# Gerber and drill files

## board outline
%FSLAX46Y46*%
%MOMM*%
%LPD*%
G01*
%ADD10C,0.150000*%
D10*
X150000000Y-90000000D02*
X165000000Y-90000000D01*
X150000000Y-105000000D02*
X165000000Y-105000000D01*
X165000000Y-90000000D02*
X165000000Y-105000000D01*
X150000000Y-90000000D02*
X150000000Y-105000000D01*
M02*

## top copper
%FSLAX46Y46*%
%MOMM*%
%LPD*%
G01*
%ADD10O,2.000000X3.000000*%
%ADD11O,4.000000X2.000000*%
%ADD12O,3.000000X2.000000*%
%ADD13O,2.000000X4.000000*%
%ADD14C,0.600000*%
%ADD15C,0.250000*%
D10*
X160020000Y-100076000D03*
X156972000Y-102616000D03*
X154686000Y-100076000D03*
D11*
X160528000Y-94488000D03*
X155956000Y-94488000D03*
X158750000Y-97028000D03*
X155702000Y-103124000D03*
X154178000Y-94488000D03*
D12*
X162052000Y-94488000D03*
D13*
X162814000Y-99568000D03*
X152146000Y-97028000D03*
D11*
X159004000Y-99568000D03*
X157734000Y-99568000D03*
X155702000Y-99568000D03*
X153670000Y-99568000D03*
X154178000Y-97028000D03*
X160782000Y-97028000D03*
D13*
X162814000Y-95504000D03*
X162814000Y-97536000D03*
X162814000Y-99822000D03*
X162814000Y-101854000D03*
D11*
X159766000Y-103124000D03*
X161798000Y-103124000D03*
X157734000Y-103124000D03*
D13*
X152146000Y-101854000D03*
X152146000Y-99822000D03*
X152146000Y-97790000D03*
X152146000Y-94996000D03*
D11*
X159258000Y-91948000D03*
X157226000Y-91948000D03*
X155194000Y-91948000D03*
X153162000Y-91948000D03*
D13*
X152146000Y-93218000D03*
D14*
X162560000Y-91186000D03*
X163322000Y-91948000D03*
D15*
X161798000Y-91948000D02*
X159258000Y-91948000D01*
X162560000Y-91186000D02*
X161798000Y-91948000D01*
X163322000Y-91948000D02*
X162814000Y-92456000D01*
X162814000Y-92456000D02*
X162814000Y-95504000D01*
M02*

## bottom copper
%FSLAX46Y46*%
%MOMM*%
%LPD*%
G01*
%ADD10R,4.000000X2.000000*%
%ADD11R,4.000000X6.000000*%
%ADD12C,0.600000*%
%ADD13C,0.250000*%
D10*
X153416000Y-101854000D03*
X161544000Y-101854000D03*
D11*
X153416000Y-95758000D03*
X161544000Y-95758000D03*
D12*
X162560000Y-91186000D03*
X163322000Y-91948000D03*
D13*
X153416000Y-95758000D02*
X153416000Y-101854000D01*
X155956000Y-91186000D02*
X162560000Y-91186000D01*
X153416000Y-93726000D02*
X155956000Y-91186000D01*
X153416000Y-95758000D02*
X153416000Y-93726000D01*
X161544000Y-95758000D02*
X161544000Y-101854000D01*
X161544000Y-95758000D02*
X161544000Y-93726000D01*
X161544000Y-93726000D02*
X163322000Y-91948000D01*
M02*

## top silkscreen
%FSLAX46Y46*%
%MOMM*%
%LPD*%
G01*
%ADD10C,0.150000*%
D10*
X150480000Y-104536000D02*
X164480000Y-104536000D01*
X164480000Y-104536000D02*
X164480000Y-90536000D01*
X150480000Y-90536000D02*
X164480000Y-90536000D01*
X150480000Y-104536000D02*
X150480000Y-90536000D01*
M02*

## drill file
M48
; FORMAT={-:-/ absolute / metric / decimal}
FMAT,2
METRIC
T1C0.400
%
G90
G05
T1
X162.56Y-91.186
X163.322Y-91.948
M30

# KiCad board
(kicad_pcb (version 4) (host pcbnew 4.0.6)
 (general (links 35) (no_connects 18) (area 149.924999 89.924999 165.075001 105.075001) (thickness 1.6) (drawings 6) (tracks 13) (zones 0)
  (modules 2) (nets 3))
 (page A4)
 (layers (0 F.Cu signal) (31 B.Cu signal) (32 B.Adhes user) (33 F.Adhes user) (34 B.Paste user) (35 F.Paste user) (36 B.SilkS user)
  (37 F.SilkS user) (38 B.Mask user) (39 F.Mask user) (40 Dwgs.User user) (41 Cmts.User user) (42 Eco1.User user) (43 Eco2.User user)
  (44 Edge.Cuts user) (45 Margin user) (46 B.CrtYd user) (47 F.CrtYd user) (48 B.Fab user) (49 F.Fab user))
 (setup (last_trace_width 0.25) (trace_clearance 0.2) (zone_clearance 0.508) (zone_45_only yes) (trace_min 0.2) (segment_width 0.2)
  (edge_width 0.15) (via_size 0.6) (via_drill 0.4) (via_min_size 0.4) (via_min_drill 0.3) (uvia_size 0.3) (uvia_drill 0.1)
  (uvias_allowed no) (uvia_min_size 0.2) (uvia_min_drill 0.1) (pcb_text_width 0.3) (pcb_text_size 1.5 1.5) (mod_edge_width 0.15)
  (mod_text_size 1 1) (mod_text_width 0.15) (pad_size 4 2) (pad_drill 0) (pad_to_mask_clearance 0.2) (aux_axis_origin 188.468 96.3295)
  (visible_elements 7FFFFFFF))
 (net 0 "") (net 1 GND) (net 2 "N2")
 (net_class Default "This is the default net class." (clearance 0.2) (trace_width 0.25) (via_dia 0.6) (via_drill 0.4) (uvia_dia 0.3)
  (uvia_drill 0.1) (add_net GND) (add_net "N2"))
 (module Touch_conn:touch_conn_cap (layer B.Cu) (at 157.48 97.79 90)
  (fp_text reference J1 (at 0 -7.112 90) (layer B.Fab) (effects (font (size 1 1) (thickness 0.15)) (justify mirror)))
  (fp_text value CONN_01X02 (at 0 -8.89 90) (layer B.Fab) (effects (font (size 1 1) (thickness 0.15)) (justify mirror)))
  (pad 2 smd rect (at -4.064 -4.064 90) (size 2 4) (layers B.Cu B.Paste B.Mask) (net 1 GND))
  (pad 1 smd rect (at -4.064 4.064 90) (size 2 4) (layers B.Cu B.Paste B.Mask) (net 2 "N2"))
  (pad 2 smd rect (at 2.032 -4.064 90) (size 6 4) (layers B.Cu B.Paste B.Mask) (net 1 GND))
  (pad 1 smd rect (at 2.032 4.064 90) (size 6 4) (layers B.Cu B.Paste B.Mask) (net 2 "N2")))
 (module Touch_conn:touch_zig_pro (layer F.Cu) (at 157.48 97.536)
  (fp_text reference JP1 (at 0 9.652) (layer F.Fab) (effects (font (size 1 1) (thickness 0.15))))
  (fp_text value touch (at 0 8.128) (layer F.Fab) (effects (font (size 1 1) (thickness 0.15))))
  (fp_line (start -7 7) (end 7 7) (layer F.SilkS) (width 0.15))
  (fp_line (start 7 7) (end 7 -7) (layer F.SilkS) (width 0.15))
  (fp_line (start -7 -7) (end 7 -7) (layer F.SilkS) (width 0.15))
  (fp_line (start -7 7) (end -7 -7) (layer F.SilkS) (width 0.15))
  (pad 1 smd oval (at 2.54 2.54) (size 2 3) (layers F.Cu F.Paste F.Mask) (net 1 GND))
  (pad 2 smd oval (at -0.508 5.08) (size 2 3) (layers F.Cu F.Paste F.Mask) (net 2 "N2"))
  (pad 1 smd oval (at -2.794 2.54) (size 2 3) (layers F.Cu F.Paste F.Mask) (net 1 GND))
  (pad 2 smd oval (at 3.048 -3.048) (size 4 2) (layers F.Cu F.Paste F.Mask) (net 2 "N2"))
  (pad 1 smd oval (at -1.524 -3.048) (size 4 2) (layers F.Cu F.Paste F.Mask) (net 1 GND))
  (pad 2 smd oval (at 1.27 -0.508) (size 4 2) (layers F.Cu F.Paste F.Mask) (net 2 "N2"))
  (pad 2 smd oval (at -1.778 5.588) (size 4 2) (layers F.Cu F.Paste F.Mask) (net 2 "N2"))
  (pad 1 smd oval (at -3.302 -3.048) (size 4 2) (layers F.Cu F.Paste F.Mask) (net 1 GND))
  (pad 2 smd oval (at 4.572 -3.048) (size 3 2) (layers F.Cu F.Paste F.Mask) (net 2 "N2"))
  (pad 2 smd oval (at 5.334 2.032) (size 2 4) (layers F.Cu F.Paste F.Mask) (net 2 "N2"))
  (pad 1 smd oval (at -5.334 -0.508) (size 2 4) (layers F.Cu F.Paste F.Mask) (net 1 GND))
  (pad 1 smd oval (at 1.524 2.032) (size 4 2) (layers F.Cu F.Paste F.Mask) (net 1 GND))
  (pad 1 smd oval (at 0.254 2.032) (size 4 2) (layers F.Cu F.Paste F.Mask) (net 1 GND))
  (pad 1 smd oval (at -1.778 2.032) (size 4 2) (layers F.Cu F.Paste F.Mask) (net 1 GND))
  (pad 1 smd oval (at -3.81 2.032) (size 4 2) (layers F.Cu F.Paste F.Mask) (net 1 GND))
  (pad 1 smd oval (at -3.302 -0.508) (size 4 2) (layers F.Cu F.Paste F.Mask) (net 1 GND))
  (pad 2 smd oval (at 3.302 -0.508) (size 4 2) (layers F.Cu F.Paste F.Mask) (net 2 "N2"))
  (pad 2 smd oval (at 5.334 -2.032) (size 2 4) (layers F.Cu F.Paste F.Mask) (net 2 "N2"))
  (pad 2 smd oval (at 5.334 0) (size 2 4) (layers F.Cu F.Paste F.Mask) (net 2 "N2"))
  (pad 2 smd oval (at 5.334 2.286) (size 2 4) (layers F.Cu F.Paste F.Mask) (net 2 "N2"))
  (pad 2 smd oval (at 5.334 4.318) (size 2 4) (layers F.Cu F.Paste F.Mask) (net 2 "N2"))
  (pad 2 smd oval (at 2.286 5.588) (size 4 2) (layers F.Cu F.Paste F.Mask) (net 2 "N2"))
  (pad 2 smd oval (at 4.318 5.588) (size 4 2) (layers F.Cu F.Paste F.Mask) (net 2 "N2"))
  (pad 2 smd oval (at 0.254 5.588) (size 4 2) (layers F.Cu F.Paste F.Mask) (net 2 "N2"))
  (pad 1 smd oval (at -5.334 4.318) (size 2 4) (layers F.Cu F.Paste F.Mask) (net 1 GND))
  (pad 1 smd oval (at -5.334 2.286) (size 2 4) (layers F.Cu F.Paste F.Mask) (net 1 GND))
  (pad 1 smd oval (at -5.334 0.254) (size 2 4) (layers F.Cu F.Paste F.Mask) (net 1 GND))
  (pad 1 smd oval (at -5.334 -2.54) (size 2 4) (layers F.Cu F.Paste F.Mask) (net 1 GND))
  (pad 1 smd oval (at 1.778 -5.588) (size 4 2) (layers F.Cu F.Paste F.Mask) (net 1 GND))
  (pad 1 smd oval (at -0.254 -5.588) (size 4 2) (layers F.Cu F.Paste F.Mask) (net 1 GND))
  (pad 1 smd oval (at -2.286 -5.588) (size 4 2) (layers F.Cu F.Paste F.Mask) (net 1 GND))
  (pad 1 smd oval (at -4.318 -5.588) (size 4 2) (layers F.Cu F.Paste F.Mask) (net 1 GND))
  (pad 1 smd oval (at -5.334 -4.318) (size 2 4) (layers F.Cu F.Paste F.Mask) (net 1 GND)))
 (gr_line (start 150 90) (end 165 90) (angle 90) (layer Edge.Cuts) (width 0.15))
 (gr_line (start 150 105) (end 165 105) (angle 90) (layer Edge.Cuts) (width 0.15))
 (gr_line (start 165 90) (end 165 105) (angle 90) (layer Edge.Cuts) (width 0.15))
 (gr_line (start 150 90) (end 150 105) (angle 90) (layer Edge.Cuts) (width 0.15))
 (segment (start 153.416 95.758) (end 153.416 101.854) (width 0.25) (layer B.Cu) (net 1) (status C00000))
 (segment (start 161.798 91.948) (end 159.258 91.948) (width 0.25) (layer F.Cu) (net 1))
 (segment (start 162.56 91.186) (end 161.798 91.948) (width 0.25) (layer F.Cu) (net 1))
 (via (at 162.56 91.186) (size 0.6) (drill 0.4) (layers F.Cu B.Cu) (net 1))
 (segment (start 155.956 91.186) (end 162.56 91.186) (width 0.25) (layer B.Cu) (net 1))
 (segment (start 153.416 93.726) (end 155.956 91.186) (width 0.25) (layer B.Cu) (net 1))
 (segment (start 153.416 95.758) (end 153.416 93.726) (width 0.25) (layer B.Cu) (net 1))
 (segment (start 161.544 95.758) (end 161.544 101.854) (width 0.25) (layer B.Cu) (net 2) (status C00000))
 (segment (start 161.544 95.758) (end 161.544 93.726) (width 0.25) (layer B.Cu) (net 2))
 (segment (start 161.544 93.726) (end 163.322 91.948) (width 0.25) (layer B.Cu) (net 2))
 (via (at 163.322 91.948) (size 0.6) (drill 0.4) (layers F.Cu B.Cu) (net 2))
 (segment (start 163.322 91.948) (end 162.814 92.456) (width 0.25) (layer F.Cu) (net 2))
 (segment (start 162.814 92.456) (end 162.814 95.504) (width 0.25) (layer F.Cu) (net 2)))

